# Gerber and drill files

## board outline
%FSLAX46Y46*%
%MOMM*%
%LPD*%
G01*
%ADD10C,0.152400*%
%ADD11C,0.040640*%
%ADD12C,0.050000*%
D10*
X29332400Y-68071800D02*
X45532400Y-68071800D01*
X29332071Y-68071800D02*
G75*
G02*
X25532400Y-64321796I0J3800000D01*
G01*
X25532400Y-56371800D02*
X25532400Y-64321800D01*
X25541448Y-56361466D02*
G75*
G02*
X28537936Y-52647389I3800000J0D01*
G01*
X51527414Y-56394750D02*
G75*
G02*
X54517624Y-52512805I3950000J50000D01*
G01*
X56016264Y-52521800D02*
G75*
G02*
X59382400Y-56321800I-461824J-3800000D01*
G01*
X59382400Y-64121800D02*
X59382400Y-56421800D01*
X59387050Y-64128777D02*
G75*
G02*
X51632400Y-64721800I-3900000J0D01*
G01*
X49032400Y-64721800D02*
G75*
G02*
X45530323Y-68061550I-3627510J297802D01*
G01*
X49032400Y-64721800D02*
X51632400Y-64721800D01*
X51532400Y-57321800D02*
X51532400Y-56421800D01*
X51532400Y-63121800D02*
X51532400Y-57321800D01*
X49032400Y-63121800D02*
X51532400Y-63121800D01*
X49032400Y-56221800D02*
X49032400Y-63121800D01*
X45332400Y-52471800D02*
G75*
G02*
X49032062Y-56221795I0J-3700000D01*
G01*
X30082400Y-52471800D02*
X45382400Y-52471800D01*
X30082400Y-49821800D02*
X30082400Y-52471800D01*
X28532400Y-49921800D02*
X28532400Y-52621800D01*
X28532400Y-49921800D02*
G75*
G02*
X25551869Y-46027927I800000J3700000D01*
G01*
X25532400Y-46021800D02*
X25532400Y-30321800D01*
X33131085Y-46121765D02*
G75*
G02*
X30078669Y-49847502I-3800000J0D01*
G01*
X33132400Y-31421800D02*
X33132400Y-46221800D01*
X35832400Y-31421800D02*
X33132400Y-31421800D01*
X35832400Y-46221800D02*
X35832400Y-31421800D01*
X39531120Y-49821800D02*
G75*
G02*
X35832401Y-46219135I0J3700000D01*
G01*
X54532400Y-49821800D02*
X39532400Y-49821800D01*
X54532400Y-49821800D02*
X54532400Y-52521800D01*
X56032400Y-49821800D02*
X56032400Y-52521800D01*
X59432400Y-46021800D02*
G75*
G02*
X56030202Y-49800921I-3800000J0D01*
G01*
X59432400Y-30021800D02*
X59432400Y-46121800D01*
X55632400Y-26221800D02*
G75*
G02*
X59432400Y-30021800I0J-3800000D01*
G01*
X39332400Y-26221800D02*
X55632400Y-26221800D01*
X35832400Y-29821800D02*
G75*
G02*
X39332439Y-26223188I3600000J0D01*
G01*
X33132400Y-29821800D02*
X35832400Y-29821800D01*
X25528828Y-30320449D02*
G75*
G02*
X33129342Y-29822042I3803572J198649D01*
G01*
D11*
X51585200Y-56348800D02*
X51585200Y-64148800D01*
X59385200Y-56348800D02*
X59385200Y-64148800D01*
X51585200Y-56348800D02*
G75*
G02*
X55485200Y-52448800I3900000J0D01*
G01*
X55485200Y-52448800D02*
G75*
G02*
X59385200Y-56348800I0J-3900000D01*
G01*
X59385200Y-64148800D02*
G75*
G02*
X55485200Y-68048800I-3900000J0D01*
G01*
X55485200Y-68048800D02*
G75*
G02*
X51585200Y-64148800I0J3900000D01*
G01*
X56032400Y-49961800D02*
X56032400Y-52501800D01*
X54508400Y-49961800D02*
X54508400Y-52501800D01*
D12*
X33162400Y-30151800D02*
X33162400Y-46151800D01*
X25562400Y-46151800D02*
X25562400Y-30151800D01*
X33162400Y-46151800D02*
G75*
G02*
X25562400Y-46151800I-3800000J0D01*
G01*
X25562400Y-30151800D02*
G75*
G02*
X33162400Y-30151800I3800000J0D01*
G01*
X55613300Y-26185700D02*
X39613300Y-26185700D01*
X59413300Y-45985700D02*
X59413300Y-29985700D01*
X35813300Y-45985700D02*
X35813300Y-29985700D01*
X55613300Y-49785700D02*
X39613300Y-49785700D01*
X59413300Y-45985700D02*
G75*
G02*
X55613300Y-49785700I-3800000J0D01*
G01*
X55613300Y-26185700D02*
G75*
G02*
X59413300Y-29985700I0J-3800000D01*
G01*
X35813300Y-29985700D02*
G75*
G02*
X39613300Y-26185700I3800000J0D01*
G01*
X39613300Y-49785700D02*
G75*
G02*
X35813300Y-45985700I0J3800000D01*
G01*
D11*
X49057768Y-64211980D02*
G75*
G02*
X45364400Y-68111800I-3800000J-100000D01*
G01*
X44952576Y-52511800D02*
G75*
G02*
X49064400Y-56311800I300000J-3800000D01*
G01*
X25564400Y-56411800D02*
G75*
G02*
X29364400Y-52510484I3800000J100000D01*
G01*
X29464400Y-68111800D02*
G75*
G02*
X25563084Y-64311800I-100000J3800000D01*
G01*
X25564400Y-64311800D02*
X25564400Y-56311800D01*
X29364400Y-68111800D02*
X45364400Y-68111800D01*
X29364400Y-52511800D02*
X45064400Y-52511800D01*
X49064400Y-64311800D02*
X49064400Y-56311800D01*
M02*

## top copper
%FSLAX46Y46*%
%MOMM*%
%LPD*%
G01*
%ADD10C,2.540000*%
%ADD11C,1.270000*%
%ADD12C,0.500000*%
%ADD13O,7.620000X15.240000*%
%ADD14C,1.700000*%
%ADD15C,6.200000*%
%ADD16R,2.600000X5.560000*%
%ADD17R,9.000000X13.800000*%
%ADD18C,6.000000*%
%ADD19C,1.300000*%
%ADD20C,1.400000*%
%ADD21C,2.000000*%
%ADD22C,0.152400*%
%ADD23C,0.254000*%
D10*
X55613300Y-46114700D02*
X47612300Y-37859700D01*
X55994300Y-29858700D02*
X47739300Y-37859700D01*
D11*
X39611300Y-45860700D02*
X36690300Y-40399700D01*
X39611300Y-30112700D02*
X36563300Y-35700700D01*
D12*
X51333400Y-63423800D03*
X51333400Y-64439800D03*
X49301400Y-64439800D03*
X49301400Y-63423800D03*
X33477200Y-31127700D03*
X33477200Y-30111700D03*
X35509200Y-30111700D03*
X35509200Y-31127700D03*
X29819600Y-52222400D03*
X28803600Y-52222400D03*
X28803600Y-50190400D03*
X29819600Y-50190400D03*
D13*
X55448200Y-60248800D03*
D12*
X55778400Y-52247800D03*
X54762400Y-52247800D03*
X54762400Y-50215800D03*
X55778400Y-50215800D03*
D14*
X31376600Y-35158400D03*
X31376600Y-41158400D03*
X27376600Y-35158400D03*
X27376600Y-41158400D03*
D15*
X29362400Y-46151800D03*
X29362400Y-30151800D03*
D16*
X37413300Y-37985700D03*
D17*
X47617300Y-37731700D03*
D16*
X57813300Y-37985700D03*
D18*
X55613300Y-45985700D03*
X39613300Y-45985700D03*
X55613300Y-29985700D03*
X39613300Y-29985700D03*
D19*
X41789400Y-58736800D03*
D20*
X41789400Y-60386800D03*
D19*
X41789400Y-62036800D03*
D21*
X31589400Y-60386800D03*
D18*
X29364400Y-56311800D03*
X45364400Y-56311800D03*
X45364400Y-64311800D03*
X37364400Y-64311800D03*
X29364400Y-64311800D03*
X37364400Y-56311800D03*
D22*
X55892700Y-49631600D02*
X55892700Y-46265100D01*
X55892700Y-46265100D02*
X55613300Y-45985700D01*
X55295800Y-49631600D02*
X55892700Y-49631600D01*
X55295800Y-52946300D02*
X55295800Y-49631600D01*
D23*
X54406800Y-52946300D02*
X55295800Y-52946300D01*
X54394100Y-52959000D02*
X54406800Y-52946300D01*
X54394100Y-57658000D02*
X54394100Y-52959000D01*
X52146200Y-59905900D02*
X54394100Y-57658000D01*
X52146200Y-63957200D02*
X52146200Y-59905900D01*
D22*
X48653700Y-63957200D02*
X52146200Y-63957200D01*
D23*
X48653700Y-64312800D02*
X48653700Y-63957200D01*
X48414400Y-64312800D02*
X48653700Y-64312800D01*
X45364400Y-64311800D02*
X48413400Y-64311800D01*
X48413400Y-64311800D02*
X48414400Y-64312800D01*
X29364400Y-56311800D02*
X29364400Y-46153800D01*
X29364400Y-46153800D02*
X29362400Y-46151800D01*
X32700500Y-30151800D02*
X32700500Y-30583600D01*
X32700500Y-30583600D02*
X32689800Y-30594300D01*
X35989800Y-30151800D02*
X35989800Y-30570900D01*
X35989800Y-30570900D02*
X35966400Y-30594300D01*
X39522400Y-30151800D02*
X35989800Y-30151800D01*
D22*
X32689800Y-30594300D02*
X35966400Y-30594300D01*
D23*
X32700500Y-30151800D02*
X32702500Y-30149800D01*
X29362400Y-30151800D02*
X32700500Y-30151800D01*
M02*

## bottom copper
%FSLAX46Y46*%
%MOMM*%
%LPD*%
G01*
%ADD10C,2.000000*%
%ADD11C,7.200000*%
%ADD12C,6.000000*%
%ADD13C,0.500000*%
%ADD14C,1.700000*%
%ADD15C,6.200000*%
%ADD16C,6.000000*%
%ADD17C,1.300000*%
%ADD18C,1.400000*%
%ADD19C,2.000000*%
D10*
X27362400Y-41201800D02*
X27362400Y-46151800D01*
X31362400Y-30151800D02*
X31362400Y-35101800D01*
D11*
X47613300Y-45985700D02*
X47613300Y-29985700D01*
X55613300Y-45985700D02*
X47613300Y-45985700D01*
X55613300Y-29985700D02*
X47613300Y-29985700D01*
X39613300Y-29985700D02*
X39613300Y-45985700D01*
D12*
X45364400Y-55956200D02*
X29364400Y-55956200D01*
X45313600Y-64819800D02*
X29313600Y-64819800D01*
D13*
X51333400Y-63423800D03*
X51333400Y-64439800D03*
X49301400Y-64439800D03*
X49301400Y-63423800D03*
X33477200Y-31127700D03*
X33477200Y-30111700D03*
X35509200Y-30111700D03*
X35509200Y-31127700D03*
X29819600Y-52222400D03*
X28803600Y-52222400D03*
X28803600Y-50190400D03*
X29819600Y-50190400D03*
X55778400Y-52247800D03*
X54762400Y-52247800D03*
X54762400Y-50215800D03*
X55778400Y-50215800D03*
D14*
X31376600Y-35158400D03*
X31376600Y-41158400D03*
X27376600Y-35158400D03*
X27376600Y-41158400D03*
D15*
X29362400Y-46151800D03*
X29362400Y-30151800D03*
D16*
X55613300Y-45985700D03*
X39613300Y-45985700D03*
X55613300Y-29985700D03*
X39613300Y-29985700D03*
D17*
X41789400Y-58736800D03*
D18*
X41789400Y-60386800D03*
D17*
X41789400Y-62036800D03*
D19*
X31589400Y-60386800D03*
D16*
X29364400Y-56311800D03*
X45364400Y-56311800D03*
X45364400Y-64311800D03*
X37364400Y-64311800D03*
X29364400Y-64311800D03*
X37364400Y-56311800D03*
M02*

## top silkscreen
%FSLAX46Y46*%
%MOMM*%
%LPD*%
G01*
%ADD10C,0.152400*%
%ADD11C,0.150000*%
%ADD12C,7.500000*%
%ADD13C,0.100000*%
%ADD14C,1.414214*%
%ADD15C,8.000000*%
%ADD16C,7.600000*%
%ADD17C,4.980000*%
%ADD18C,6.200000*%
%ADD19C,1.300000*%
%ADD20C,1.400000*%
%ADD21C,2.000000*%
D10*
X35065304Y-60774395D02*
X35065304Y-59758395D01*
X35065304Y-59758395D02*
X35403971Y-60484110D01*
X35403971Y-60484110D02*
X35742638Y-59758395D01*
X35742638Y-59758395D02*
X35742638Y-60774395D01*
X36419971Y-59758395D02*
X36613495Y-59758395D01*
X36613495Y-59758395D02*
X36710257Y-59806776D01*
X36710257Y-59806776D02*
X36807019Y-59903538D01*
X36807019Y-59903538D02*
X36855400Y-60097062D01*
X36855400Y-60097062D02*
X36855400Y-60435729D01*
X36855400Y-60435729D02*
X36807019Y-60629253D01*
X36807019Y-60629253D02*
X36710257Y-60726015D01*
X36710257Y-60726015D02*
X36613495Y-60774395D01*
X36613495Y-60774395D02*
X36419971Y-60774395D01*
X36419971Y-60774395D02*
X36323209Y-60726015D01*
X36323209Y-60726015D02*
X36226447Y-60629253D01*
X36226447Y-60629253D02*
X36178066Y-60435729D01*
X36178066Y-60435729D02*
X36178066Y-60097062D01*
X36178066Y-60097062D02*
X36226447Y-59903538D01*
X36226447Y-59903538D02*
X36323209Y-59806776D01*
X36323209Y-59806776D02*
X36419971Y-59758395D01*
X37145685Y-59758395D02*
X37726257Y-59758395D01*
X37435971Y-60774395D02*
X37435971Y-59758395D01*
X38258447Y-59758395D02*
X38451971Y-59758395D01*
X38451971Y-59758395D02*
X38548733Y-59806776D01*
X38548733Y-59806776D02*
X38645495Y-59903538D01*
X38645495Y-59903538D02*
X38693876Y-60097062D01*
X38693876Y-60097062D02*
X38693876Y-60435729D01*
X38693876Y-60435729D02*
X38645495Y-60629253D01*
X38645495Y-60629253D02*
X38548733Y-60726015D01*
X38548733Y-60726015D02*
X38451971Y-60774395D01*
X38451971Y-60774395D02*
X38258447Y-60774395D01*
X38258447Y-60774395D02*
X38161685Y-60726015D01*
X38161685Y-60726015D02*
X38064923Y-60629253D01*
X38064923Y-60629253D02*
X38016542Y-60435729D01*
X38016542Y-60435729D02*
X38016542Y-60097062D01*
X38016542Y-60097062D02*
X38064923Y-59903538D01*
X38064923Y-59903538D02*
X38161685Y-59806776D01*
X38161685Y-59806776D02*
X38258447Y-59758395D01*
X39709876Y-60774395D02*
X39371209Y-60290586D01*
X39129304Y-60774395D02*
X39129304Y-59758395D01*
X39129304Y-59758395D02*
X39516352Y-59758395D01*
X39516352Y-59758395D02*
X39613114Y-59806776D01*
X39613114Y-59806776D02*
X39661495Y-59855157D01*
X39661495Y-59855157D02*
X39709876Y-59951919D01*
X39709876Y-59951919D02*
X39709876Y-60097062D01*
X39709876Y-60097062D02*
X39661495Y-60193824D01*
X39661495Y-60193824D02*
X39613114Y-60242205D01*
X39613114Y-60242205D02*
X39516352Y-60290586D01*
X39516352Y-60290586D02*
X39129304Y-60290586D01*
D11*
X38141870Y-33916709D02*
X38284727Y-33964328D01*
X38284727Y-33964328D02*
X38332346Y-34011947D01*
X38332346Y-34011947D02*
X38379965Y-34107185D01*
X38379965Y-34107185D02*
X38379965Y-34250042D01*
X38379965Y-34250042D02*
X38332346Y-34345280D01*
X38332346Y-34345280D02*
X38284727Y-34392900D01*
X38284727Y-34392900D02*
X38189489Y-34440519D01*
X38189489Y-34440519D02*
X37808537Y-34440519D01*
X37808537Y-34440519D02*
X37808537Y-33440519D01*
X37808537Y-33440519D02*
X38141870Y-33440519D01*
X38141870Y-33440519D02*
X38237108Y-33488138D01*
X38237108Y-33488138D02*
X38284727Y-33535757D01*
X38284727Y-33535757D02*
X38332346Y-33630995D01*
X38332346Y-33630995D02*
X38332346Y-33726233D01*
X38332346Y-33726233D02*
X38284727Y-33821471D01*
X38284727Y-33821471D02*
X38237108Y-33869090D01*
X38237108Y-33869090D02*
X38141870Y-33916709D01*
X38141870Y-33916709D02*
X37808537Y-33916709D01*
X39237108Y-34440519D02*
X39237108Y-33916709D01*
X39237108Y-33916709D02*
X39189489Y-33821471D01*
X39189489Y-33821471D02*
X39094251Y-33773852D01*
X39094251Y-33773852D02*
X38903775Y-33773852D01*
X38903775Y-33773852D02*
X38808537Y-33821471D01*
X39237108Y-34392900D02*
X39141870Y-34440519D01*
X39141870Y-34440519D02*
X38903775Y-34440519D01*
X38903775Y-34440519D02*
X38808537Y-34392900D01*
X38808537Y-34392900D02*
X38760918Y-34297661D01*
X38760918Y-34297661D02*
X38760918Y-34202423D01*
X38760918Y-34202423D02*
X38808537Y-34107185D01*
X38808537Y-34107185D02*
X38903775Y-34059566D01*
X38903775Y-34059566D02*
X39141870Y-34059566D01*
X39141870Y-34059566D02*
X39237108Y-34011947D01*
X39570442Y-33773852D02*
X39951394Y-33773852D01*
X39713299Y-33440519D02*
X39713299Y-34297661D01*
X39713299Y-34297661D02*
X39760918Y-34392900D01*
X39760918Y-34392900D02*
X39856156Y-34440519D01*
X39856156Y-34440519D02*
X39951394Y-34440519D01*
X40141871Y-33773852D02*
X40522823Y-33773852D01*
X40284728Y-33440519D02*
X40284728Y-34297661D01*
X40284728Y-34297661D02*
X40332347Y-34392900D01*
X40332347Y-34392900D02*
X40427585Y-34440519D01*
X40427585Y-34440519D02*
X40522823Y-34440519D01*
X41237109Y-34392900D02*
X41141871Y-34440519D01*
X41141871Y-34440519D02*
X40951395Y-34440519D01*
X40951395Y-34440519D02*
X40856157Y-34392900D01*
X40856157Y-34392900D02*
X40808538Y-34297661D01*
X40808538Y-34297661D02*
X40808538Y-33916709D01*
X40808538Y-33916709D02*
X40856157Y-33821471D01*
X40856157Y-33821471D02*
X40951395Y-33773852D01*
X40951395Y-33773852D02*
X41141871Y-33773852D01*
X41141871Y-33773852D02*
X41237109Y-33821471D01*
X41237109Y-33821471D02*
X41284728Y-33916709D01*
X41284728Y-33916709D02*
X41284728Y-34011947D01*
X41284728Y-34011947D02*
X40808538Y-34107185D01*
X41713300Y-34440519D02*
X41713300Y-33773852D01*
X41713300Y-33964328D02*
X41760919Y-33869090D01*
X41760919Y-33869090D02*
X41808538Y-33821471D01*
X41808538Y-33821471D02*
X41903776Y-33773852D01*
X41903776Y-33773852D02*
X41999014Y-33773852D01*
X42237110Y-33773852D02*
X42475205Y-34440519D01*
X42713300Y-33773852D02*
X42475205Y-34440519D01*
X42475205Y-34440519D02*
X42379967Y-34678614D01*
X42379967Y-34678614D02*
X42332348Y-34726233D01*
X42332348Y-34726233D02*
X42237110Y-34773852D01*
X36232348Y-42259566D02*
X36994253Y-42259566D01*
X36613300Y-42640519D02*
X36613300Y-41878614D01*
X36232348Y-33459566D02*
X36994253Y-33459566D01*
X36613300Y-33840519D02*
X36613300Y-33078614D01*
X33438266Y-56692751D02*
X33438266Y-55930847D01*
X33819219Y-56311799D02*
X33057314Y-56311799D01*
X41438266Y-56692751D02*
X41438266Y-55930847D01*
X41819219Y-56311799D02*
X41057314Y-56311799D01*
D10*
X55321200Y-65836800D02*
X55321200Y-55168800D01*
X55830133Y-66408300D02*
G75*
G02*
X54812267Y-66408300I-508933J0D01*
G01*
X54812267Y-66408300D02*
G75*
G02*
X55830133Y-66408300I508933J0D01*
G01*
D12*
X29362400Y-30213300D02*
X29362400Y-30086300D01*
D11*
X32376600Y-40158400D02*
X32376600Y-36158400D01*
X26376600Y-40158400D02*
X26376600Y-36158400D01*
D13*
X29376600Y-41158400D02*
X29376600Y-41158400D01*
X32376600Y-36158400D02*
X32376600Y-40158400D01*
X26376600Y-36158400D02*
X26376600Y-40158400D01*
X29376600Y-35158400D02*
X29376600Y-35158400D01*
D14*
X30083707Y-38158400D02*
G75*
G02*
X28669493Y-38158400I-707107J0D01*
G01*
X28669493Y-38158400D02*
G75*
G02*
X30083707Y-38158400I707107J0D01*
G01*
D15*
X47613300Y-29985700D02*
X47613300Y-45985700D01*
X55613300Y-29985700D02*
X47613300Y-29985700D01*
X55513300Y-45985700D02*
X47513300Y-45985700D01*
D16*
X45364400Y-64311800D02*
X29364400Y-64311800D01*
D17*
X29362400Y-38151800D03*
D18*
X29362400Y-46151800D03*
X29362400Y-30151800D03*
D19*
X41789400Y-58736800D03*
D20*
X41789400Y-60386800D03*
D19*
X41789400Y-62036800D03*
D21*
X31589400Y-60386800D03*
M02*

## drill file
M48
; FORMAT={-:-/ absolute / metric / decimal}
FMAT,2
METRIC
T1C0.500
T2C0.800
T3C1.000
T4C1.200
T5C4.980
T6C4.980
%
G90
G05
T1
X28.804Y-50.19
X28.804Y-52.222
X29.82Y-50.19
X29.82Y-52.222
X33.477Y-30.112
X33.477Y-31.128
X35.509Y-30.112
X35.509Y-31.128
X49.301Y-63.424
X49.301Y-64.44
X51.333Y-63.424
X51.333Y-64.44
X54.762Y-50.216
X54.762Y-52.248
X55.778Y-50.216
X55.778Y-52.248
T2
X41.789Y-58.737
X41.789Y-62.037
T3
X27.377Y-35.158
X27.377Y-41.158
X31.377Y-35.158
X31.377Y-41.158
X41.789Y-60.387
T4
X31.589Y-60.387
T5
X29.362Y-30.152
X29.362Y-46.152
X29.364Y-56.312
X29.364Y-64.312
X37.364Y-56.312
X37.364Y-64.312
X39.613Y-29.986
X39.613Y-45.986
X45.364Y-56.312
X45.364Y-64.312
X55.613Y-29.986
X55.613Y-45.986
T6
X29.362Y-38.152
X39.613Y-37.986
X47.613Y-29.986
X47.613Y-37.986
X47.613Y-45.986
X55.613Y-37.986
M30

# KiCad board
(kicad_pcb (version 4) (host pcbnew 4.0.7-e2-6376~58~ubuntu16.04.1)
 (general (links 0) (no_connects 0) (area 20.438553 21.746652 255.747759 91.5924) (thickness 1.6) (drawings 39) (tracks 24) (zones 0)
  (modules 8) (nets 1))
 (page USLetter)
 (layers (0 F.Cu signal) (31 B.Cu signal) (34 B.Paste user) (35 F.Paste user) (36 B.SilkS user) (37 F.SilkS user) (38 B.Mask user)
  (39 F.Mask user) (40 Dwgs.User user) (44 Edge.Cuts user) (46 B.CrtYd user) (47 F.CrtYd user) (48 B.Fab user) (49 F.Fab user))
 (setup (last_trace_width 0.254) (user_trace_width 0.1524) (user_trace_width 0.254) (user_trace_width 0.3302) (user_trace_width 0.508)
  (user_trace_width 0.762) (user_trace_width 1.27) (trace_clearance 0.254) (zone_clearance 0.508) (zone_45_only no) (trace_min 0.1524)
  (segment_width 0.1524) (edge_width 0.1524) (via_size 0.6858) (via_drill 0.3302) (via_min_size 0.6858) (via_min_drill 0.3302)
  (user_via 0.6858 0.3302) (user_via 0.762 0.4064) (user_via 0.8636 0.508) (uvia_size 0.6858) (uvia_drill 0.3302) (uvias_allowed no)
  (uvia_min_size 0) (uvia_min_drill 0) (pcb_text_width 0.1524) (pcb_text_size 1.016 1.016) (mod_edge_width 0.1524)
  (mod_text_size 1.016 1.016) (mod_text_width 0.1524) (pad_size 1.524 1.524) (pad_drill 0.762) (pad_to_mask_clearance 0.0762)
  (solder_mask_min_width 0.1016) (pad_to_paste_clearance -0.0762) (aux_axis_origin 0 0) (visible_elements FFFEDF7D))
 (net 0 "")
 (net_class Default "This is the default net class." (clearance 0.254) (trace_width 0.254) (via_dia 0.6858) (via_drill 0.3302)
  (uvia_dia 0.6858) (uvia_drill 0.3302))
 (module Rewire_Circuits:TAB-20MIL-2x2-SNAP (layer F.Cu) (at 50.3174 63.9318 270)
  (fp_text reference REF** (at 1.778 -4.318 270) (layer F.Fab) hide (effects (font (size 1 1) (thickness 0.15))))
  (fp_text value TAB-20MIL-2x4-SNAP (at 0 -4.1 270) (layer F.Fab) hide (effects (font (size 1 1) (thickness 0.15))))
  (pad 1 thru_hole circle (at -0.508 -1.016 270) (size 0.5 0.5) (drill 0.5) (layers *.Cu))
  (pad 1 thru_hole circle (at 0.508 -1.016 270) (size 0.5 0.5) (drill 0.5) (layers *.Cu))
  (pad 1 thru_hole circle (at 0.508 1.016 270) (size 0.5 0.5) (drill 0.5) (layers *.Cu))
  (pad 1 thru_hole circle (at -0.508 1.016 270) (size 0.5 0.5) (drill 0.5) (layers *.Cu)))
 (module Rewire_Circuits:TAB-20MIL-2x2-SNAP (layer F.Cu) (at 34.4932 30.6197 90)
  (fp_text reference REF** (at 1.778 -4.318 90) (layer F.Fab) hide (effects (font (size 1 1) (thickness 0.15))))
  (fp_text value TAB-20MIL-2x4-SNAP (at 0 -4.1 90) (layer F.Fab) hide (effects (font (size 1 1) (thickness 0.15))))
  (pad 1 thru_hole circle (at -0.508 -1.016 90) (size 0.5 0.5) (drill 0.5) (layers *.Cu))
  (pad 1 thru_hole circle (at 0.508 -1.016 90) (size 0.5 0.5) (drill 0.5) (layers *.Cu))
  (pad 1 thru_hole circle (at 0.508 1.016 90) (size 0.5 0.5) (drill 0.5) (layers *.Cu))
  (pad 1 thru_hole circle (at -0.508 1.016 90) (size 0.5 0.5) (drill 0.5) (layers *.Cu)))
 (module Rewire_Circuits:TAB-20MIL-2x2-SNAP (layer F.Cu) (at 29.3116 51.2064 180)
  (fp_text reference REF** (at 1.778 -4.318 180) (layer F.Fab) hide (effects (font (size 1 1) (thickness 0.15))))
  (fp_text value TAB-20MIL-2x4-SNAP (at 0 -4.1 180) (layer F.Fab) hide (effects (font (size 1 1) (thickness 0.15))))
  (pad 1 thru_hole circle (at -0.508 -1.016 180) (size 0.5 0.5) (drill 0.5) (layers *.Cu))
  (pad 1 thru_hole circle (at 0.508 -1.016 180) (size 0.5 0.5) (drill 0.5) (layers *.Cu))
  (pad 1 thru_hole circle (at 0.508 1.016 180) (size 0.5 0.5) (drill 0.5) (layers *.Cu))
  (pad 1 thru_hole circle (at -0.508 1.016 180) (size 0.5 0.5) (drill 0.5) (layers *.Cu)))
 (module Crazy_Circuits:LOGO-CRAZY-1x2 (layer F.Cu) (at 59.3852 60.2488 90)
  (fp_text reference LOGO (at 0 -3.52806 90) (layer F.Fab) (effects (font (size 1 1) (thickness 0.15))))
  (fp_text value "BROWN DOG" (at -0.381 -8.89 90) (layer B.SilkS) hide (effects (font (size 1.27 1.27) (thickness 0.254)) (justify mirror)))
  (fp_line (start -5.588 -4.064) (end 5.08 -4.064) (layer F.SilkS) (width 0.1524))
  (fp_circle (center -6.1595 -4.064) (end -5.82208 -3.683) (layer F.SilkS) (width 0.1524))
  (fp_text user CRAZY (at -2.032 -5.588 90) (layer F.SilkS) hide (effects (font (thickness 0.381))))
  (fp_line (start 3.9 -7.8) (end -3.9 -7.8) (layer Edge.Cuts) (width 0.04064))
  (fp_line (start 3.9 0) (end -3.9 0) (layer Edge.Cuts) (width 0.04064))
  (fp_arc (start 3.9 -3.9) (end 3.9 -7.8) (angle 90) (layer Edge.Cuts) (width 0.04064))
  (fp_arc (start 3.9 -3.9) (end 7.8 -3.9) (angle 90) (layer Edge.Cuts) (width 0.04064))
  (fp_arc (start -3.9 -3.9) (end -3.9 0) (angle 90) (layer Edge.Cuts) (width 0.04064))
  (fp_arc (start -3.9 -3.9) (end -7.8 -3.9) (angle 90) (layer Edge.Cuts) (width 0.04064))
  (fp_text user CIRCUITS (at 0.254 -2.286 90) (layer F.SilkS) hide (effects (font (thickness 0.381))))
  (pad BG smd oval (at 0 -3.937 90) (size 15.24 7.62) (layers F.Cu)))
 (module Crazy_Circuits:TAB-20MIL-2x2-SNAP (layer F.Cu) (at 55.2704 51.2318 180)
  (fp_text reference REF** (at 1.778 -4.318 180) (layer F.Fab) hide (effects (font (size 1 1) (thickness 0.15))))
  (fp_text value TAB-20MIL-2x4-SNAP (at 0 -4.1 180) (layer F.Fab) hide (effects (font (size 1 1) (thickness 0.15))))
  (fp_line (start -0.762 1.27) (end -0.762 -1.27) (layer Edge.Cuts) (width 0.04064))
  (fp_line (start 0.762 1.27) (end 0.762 -1.27) (layer Edge.Cuts) (width 0.04064))
  (pad 1 thru_hole circle (at -0.508 -1.016 180) (size 0.5 0.5) (drill 0.5) (layers *.Cu))
  (pad 1 thru_hole circle (at 0.508 -1.016 180) (size 0.5 0.5) (drill 0.5) (layers *.Cu))
  (pad 1 thru_hole circle (at 0.508 1.016 180) (size 0.5 0.5) (drill 0.5) (layers *.Cu))
  (pad 1 thru_hole circle (at -0.508 1.016 180) (size 0.5 0.5) (drill 0.5) (layers *.Cu)))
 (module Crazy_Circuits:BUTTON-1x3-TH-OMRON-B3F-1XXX (layer F.Cu) (at 29.3624 46.1518 90)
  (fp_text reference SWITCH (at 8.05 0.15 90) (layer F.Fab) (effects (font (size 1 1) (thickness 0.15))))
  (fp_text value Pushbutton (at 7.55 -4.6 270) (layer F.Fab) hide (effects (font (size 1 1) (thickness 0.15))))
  (fp_line (start 15.9385 0) (end 16.0655 0) (layer F.SilkS) (width 7.5))
  (fp_line (start 16 3.8) (end 0 3.8) (layer Edge.Cuts) (width 0.05))
  (fp_line (start 0 -3.8) (end 16 -3.8) (layer Edge.Cuts) (width 0.05))
  (fp_arc (start 0 0) (end 0 3.8) (angle 180) (layer Edge.Cuts) (width 0.05)) (fp_line (start 4.95 -2) (end 0 -2) (layer B.Cu) (width 2))
  (fp_line (start 5.9934 3.0142) (end 9.9934 3.0142) (layer F.SilkS) (width 0.15))
  (fp_line (start 5.9934 -2.9858) (end 9.9934 -2.9858) (layer F.SilkS) (width 0.15))
  (fp_line (start 4.9934 0.0142) (end 4.9934 0.0142) (layer F.SilkS) (width 0))
  (fp_line (start 9.9934 3.0142) (end 5.9934 3.0142) (layer F.SilkS) (width 0))
  (fp_line (start 9.9934 -2.9858) (end 5.9934 -2.9858) (layer F.SilkS) (width 0))
  (fp_line (start 10.9934 0.0142) (end 10.9934 0.0142) (layer F.SilkS) (width 0))
  (fp_circle (center 7.9934 0.0142) (end 8.9934 1.0142) (layer F.SilkS) (width 0))
  (fp_line (start 16 2) (end 11.05 2) (layer B.Cu) (width 2))
  (fp_arc (start 16 0) (end 16 -3.8) (angle 180) (layer Edge.Cuts) (width 0.05))
  (pad 2 thru_hole circle (at 10.9934 2.0142 90) (size 1.7 1.7) (drill 1) (layers *.Cu *.Mask))
  (pad 2 thru_hole circle (at 4.9934 2.0142 90) (size 1.7 1.7) (drill 1) (layers *.Cu *.Mask))
  (pad 1 thru_hole circle (at 10.9934 -1.9858 90) (size 1.7 1.7) (drill 1) (layers *.Cu *.Mask))
  (pad 1 thru_hole circle (at 4.9934 -1.9858 90) (size 1.7 1.7) (drill 1) (layers *.Cu *.Mask))
  (pad "" np_thru_hole circle (at 8 0 90) (size 4.98 4.98) (drill 4.98) (layers *.Cu F.SilkS))
  (pad 1 thru_hole circle (at 0 0 90) (size 6.2 6.2) (drill 4.98) (layers *.Cu *.Mask F.SilkS))
  (pad 2 thru_hole circle (at 16 0 90) (size 6.2 6.2) (drill 4.98) (layers *.Cu *.Mask F.SilkS)))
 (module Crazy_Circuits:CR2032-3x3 (layer F.Cu) (at 55.6133 29.9857 180)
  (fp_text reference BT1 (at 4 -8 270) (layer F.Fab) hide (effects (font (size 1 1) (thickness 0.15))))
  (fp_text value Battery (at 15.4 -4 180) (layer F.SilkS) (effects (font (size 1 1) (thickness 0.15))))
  (fp_line (start 0 -16.129) (end 8.001 -7.874) (layer F.Cu) (width 2.54))
  (fp_line (start 0 3.8) (end 16 3.8) (layer Edge.Cuts) (width 0.05))
  (fp_line (start -3.8 -16) (end -3.8 0) (layer Edge.Cuts) (width 0.05))
  (fp_line (start 19.8 -16) (end 19.8 0) (layer Edge.Cuts) (width 0.05))
  (fp_line (start 0 -19.8) (end 16 -19.8) (layer Edge.Cuts) (width 0.05))
  (fp_arc (start 0 -16) (end -3.8 -16) (angle 90) (layer Edge.Cuts) (width 0.05))
  (fp_arc (start 0 0) (end 0 3.8) (angle 90) (layer Edge.Cuts) (width 0.05))
  (fp_arc (start 16 0) (end 19.8 0) (angle 90) (layer Edge.Cuts) (width 0.05))
  (fp_arc (start 16 -16) (end 16 -19.8) (angle 90) (layer Edge.Cuts) (width 0.05))
  (fp_line (start 8 0) (end 8 -16) (layer F.SilkS) (width 8)) (fp_line (start 8 -16) (end 8 0) (layer B.Cu) (width 7.2))
  (fp_line (start 0 -16) (end 8 -16) (layer B.Cu) (width 7.2)) (fp_line (start 0 0) (end 8 0) (layer B.Cu) (width 7.2))
  (fp_line (start 16 0) (end 16 -16) (layer B.Cu) (width 7.2))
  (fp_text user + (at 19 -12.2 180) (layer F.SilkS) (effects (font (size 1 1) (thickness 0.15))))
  (fp_line (start 0 0) (end 8 0) (layer F.SilkS) (width 8))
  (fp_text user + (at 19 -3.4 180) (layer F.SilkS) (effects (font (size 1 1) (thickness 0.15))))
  (fp_line (start 0.1 -16) (end 8.1 -16) (layer F.SilkS) (width 8))
  (fp_line (start -0.381 0.127) (end 7.874 -7.874) (layer F.Cu) (width 2.54))
  (fp_line (start 16.002 -15.875) (end 18.923 -10.414) (layer F.Cu) (width 1.27))
  (fp_line (start 16.002 -0.127) (end 19.05 -5.715) (layer F.Cu) (width 1.27))
  (pad "" np_thru_hole circle (at 8 -8 180) (size 4.98 4.98) (drill 4.98) (layers *.Cu B.Mask))
  (pad "" np_thru_hole circle (at 0 -8 180) (size 4.98 4.98) (drill 4.98) (layers *.Cu B.Mask))
  (pad "" np_thru_hole circle (at 16 -8 180) (size 4.98 4.98) (drill 4.98) (layers *.Cu B.Mask))
  (pad + smd rect (at 18.2 -8 180) (size 2.6 5.56) (layers F.Cu F.Paste F.Mask))
  (pad GND smd rect (at 7.996 -7.746 180) (size 9 13.8) (layers F.Cu F.Paste F.Mask))
  (pad + smd rect (at -2.2 -8 180) (size 2.6 5.56) (layers F.Cu F.Paste F.Mask))
  (pad GND thru_hole circle (at 0 -16 180) (size 6 6) (drill 4.98) (layers *.Cu B.Mask))
  (pad "" np_thru_hole circle (at 8 -16 180) (size 4.98 4.98) (drill 4.98) (layers *.Cu B.Mask))
  (pad + thru_hole circle (at 16 -16 180) (size 6 6) (drill 4.98) (layers *.Cu B.Mask))
  (pad GND thru_hole circle (at 0 0 180) (size 6 6) (drill 4.98) (layers *.Cu B.Mask))
  (pad "" np_thru_hole circle (at 8 0 180) (size 4.98 4.98) (drill 4.98) (layers *.Cu B.Mask))
  (pad + thru_hole circle (at 16 0 180) (size 6 6) (drill 4.98) (layers *.Cu B.Mask)))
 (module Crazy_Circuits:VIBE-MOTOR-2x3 (layer F.Cu) (at 45.3644 56.3118 180)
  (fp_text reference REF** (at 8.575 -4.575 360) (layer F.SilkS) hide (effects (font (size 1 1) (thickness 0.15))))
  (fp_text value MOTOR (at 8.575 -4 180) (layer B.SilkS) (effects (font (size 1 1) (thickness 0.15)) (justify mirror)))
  (fp_line (start 0 0.3556) (end 16 0.3556) (layer B.Cu) (width 6))
  (fp_line (start 0.0508 -8.508) (end 16.0508 -8.508) (layer B.Cu) (width 6))
  (fp_line (start 0 -8) (end 16 -8) (layer F.SilkS) (width 7.6))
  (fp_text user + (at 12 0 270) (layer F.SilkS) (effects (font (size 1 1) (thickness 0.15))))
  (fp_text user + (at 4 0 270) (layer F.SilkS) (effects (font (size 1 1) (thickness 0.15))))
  (fp_arc (start 0.106632 -8.00018) (end -3.693368 -7.90018) (angle 89.9) (layer Edge.Cuts) (width 0.04064))
  (fp_arc (start 0.111824 0) (end 0.411824 3.8) (angle 94.51398846) (layer Edge.Cuts) (width 0.04064))
  (fp_arc (start 16 0) (end 19.8 -0.1) (angle 91.50743576) (layer Edge.Cuts) (width 0.04064))
  (fp_arc (start 16 -8) (end 15.9 -11.8) (angle 91.50743576) (layer Edge.Cuts) (width 0.04064))
  (fp_line (start 19.8 -8) (end 19.8 0) (layer Edge.Cuts) (width 0.04064))
  (fp_line (start 16 -11.8) (end 0 -11.8) (layer Edge.Cuts) (width 0.04064))
  (fp_line (start 16 3.8) (end 0.3 3.8) (layer Edge.Cuts) (width 0.04064))
  (fp_line (start -3.7 -8) (end -3.7 0) (layer Edge.Cuts) (width 0.04064))
  (pad 1 thru_hole circle (at 3.575 -2.425 270) (size 1.3 1.3) (drill 0.8) (layers *.Cu *.Mask F.SilkS))
  (pad 3 thru_hole circle (at 3.575 -4.075 270) (size 1.4 1.4) (drill 1) (layers *.Cu *.Mask F.SilkS))
  (pad 2 thru_hole circle (at 3.575 -5.725 270) (size 1.3 1.3) (drill 0.8) (layers *.Cu *.Mask F.SilkS))
  (pad 3 thru_hole circle (at 13.775 -4.075 270) (size 2 2) (drill 1.2) (layers *.Cu *.Mask F.SilkS))
  (pad 1 thru_hole circle (at 16 0 180) (size 6 6) (drill 4.98) (layers *.Cu *.Mask))
  (pad 1 thru_hole circle (at 0 0 180) (size 6 6) (drill 4.98) (layers *.Cu *.Mask))
  (pad 2 thru_hole circle (at 0 -8 180) (size 6 6) (drill 4.98) (layers *.Cu *.Mask))
  (pad 2 thru_hole circle (at 8 -8 180) (size 6 6) (drill 4.98) (layers *.Cu *.Mask))
  (pad 2 thru_hole circle (at 16 -8 180) (size 6 6) (drill 4.98) (layers *.Cu *.Mask))
  (pad 1 thru_hole circle (at 8 0 180) (size 6 6) (drill 4.98) (layers *.Cu *.Mask)))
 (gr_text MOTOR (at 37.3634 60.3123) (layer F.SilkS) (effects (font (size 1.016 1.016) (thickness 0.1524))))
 (gr_line (start 29.3324 68.0718) (end 45.5324 68.0718) (layer Edge.Cuts) (width 0.1524))
 (gr_arc (start 29.332071 64.2718) (end 29.332071 68.0718) (angle 89.24615167) (layer Edge.Cuts) (width 0.1524))
 (gr_line (start 25.5324 56.3718) (end 25.5324 64.3218) (layer Edge.Cuts) (width 0.1524))
 (gr_arc (start 29.341448 56.361466) (end 25.541448 56.361466) (angle 77.79262944) (layer Edge.Cuts) (width 0.1524))
 (gr_arc (start 55.477414 56.34475) (end 51.527414 56.39475) (angle 76.66359666) (layer Edge.Cuts) (width 0.1524))
 (gr_arc (start 55.55444 56.3218) (end 56.016264 52.5218) (angle 83.07067559) (layer Edge.Cuts) (width 0.1524))
 (gr_line (start 59.3824 64.1218) (end 59.3824 56.4218) (layer Edge.Cuts) (width 0.1524))
 (gr_arc (start 55.48705 64.128777) (end 59.38705 64.128777) (angle 171.2538377) (layer Edge.Cuts) (width 0.1524))
 (gr_arc (start 45.40489 64.423998) (end 49.0324 64.7218) (angle 83.33186569) (layer Edge.Cuts) (width 0.1524))
 (gr_line (start 49.0324 64.7218) (end 51.6324 64.7218) (layer Edge.Cuts) (width 0.1524))
 (gr_line (start 51.5324 57.3218) (end 51.5324 56.4218) (layer Edge.Cuts) (width 0.1524))
 (gr_line (start 51.5324 63.1218) (end 51.5324 57.3218) (layer Edge.Cuts) (width 0.1524))
 (gr_line (start 49.0324 63.1218) (end 51.5324 63.1218) (layer Edge.Cuts) (width 0.1524))
 (gr_line (start 49.0324 56.2218) (end 49.0324 63.1218) (layer Edge.Cuts) (width 0.1524))
 (gr_arc (start 45.3324 56.1718) (end 45.3324 52.4718) (angle 90.77421347) (layer Edge.Cuts) (width 0.1524))
 (gr_line (start 30.0824 52.4718) (end 45.3824 52.4718) (layer Edge.Cuts) (width 0.1524))
 (gr_line (start 30.0824 49.8218) (end 30.0824 52.4718) (layer Edge.Cuts) (width 0.1524))
 (gr_line (start 28.5324 49.9218) (end 28.5324 52.6218) (layer Edge.Cuts) (width 0.1524))
 (gr_arc (start 29.3324 46.2218) (end 28.5324 49.9218) (angle 80.73520472) (layer Edge.Cuts) (width 0.1524))
 (gr_line (start 25.5324 46.0218) (end 25.5324 30.3218) (layer Edge.Cuts) (width 0.1524))
 (gr_arc (start 29.331085 46.121765) (end 33.131085 46.121765) (angle 78.6540423) (layer Edge.Cuts) (width 0.1524))
 (gr_line (start 33.1324 31.4218) (end 33.1324 46.2218) (layer Edge.Cuts) (width 0.1524))
 (gr_line (start 35.8324 31.4218) (end 33.1324 31.4218) (layer Edge.Cuts) (width 0.1524))
 (gr_line (start 35.8324 46.2218) (end 35.8324 31.4218) (layer Edge.Cuts) (width 0.1524))
 (gr_arc (start 39.53112 46.1218) (end 39.53112 49.8218) (angle 88.49256424) (layer Edge.Cuts) (width 0.1524))
 (gr_line (start 54.5324 49.8218) (end 39.5324 49.8218) (layer Edge.Cuts) (width 0.1524))
 (gr_line (start 54.5324 49.8218) (end 54.5324 52.5218) (layer Edge.Cuts) (width 0.1524))
 (gr_line (start 56.0324 49.8218) (end 56.0324 52.5218) (layer Edge.Cuts) (width 0.1524))
 (gr_arc (start 55.6324 46.0218) (end 59.4324 46.0218) (angle 83.99099562) (layer Edge.Cuts) (width 0.1524))
 (gr_line (start 59.4324 30.0218) (end 59.4324 46.1218) (layer Edge.Cuts) (width 0.1524))
 (gr_arc (start 55.6324 30.0218) (end 55.6324 26.2218) (angle 90) (layer Edge.Cuts) (width 0.1524))
 (gr_line (start 39.3324 26.2218) (end 55.6324 26.2218) (layer Edge.Cuts) (width 0.1524))
 (gr_arc (start 39.4324 29.8218) (end 35.8324 29.8218) (angle 88.40885973) (layer Edge.Cuts) (width 0.1524))
 (gr_line (start 33.1324 29.8218) (end 35.8324 29.8218) (layer Edge.Cuts) (width 0.1524))
 (gr_arc (start 29.3324 30.1218) (end 25.528828 30.320449) (angle 178.4756859) (layer Edge.Cuts) (width 0.1524))
 (segment (start 55.8927 49.6316) (end 55.8927 46.2651) (width 0.1524) (layer F.Cu) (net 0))
 (segment (start 55.8927 46.2651) (end 55.6133 45.9857) (width 0.1524) (layer F.Cu) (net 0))
 (segment (start 55.2958 49.6316) (end 55.8927 49.6316) (width 0.1524) (layer F.Cu) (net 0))
 (segment (start 55.2958 52.9463) (end 55.2958 49.6316) (width 0.1524) (layer F.Cu) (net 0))
 (segment (start 54.4068 52.9463) (end 55.2958 52.9463) (width 0.254) (layer F.Cu) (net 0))
 (segment (start 54.3941 52.959) (end 54.4068 52.9463) (width 0.254) (layer F.Cu) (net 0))
 (segment (start 54.3941 57.658) (end 54.3941 52.959) (width 0.254) (layer F.Cu) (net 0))
 (segment (start 52.1462 59.9059) (end 54.3941 57.658) (width 0.254) (layer F.Cu) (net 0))
 (segment (start 52.1462 63.9572) (end 52.1462 59.9059) (width 0.254) (layer F.Cu) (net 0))
 (segment (start 48.6537 63.9572) (end 52.1462 63.9572) (width 0.1524) (layer F.Cu) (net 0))
 (segment (start 48.6537 64.3128) (end 48.6537 63.9572) (width 0.254) (layer F.Cu) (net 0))
 (segment (start 48.4144 64.3128) (end 48.6537 64.3128) (width 0.254) (layer F.Cu) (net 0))
 (segment (start 45.3644 64.3118) (end 48.4134 64.3118) (width 0.254) (layer F.Cu) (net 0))
 (segment (start 48.4134 64.3118) (end 48.4144 64.3128) (width 0.254) (layer F.Cu) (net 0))
 (segment (start 29.3644 56.3118) (end 29.3644 46.1538) (width 0.254) (layer F.Cu) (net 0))
 (segment (start 29.3644 46.1538) (end 29.3624 46.1518) (width 0.254) (layer F.Cu) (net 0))
 (segment (start 32.7005 30.1518) (end 32.7005 30.5836) (width 0.254) (layer F.Cu) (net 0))
 (segment (start 32.7005 30.5836) (end 32.6898 30.5943) (width 0.254) (layer F.Cu) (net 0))
 (segment (start 35.9898 30.1518) (end 35.9898 30.5709) (width 0.254) (layer F.Cu) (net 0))
 (segment (start 35.9898 30.5709) (end 35.9664 30.5943) (width 0.254) (layer F.Cu) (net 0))
 (segment (start 39.5224 30.1518) (end 35.9898 30.1518) (width 0.254) (layer F.Cu) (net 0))
 (segment (start 32.6898 30.5943) (end 35.9664 30.5943) (width 0.1524) (layer F.Cu) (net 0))
 (segment (start 32.7005 30.1518) (end 32.7025 30.1498) (width 0.254) (layer F.Cu) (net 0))
 (segment (start 29.3624 30.1518) (end 32.7005 30.1518) (width 0.254) (layer F.Cu) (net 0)))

